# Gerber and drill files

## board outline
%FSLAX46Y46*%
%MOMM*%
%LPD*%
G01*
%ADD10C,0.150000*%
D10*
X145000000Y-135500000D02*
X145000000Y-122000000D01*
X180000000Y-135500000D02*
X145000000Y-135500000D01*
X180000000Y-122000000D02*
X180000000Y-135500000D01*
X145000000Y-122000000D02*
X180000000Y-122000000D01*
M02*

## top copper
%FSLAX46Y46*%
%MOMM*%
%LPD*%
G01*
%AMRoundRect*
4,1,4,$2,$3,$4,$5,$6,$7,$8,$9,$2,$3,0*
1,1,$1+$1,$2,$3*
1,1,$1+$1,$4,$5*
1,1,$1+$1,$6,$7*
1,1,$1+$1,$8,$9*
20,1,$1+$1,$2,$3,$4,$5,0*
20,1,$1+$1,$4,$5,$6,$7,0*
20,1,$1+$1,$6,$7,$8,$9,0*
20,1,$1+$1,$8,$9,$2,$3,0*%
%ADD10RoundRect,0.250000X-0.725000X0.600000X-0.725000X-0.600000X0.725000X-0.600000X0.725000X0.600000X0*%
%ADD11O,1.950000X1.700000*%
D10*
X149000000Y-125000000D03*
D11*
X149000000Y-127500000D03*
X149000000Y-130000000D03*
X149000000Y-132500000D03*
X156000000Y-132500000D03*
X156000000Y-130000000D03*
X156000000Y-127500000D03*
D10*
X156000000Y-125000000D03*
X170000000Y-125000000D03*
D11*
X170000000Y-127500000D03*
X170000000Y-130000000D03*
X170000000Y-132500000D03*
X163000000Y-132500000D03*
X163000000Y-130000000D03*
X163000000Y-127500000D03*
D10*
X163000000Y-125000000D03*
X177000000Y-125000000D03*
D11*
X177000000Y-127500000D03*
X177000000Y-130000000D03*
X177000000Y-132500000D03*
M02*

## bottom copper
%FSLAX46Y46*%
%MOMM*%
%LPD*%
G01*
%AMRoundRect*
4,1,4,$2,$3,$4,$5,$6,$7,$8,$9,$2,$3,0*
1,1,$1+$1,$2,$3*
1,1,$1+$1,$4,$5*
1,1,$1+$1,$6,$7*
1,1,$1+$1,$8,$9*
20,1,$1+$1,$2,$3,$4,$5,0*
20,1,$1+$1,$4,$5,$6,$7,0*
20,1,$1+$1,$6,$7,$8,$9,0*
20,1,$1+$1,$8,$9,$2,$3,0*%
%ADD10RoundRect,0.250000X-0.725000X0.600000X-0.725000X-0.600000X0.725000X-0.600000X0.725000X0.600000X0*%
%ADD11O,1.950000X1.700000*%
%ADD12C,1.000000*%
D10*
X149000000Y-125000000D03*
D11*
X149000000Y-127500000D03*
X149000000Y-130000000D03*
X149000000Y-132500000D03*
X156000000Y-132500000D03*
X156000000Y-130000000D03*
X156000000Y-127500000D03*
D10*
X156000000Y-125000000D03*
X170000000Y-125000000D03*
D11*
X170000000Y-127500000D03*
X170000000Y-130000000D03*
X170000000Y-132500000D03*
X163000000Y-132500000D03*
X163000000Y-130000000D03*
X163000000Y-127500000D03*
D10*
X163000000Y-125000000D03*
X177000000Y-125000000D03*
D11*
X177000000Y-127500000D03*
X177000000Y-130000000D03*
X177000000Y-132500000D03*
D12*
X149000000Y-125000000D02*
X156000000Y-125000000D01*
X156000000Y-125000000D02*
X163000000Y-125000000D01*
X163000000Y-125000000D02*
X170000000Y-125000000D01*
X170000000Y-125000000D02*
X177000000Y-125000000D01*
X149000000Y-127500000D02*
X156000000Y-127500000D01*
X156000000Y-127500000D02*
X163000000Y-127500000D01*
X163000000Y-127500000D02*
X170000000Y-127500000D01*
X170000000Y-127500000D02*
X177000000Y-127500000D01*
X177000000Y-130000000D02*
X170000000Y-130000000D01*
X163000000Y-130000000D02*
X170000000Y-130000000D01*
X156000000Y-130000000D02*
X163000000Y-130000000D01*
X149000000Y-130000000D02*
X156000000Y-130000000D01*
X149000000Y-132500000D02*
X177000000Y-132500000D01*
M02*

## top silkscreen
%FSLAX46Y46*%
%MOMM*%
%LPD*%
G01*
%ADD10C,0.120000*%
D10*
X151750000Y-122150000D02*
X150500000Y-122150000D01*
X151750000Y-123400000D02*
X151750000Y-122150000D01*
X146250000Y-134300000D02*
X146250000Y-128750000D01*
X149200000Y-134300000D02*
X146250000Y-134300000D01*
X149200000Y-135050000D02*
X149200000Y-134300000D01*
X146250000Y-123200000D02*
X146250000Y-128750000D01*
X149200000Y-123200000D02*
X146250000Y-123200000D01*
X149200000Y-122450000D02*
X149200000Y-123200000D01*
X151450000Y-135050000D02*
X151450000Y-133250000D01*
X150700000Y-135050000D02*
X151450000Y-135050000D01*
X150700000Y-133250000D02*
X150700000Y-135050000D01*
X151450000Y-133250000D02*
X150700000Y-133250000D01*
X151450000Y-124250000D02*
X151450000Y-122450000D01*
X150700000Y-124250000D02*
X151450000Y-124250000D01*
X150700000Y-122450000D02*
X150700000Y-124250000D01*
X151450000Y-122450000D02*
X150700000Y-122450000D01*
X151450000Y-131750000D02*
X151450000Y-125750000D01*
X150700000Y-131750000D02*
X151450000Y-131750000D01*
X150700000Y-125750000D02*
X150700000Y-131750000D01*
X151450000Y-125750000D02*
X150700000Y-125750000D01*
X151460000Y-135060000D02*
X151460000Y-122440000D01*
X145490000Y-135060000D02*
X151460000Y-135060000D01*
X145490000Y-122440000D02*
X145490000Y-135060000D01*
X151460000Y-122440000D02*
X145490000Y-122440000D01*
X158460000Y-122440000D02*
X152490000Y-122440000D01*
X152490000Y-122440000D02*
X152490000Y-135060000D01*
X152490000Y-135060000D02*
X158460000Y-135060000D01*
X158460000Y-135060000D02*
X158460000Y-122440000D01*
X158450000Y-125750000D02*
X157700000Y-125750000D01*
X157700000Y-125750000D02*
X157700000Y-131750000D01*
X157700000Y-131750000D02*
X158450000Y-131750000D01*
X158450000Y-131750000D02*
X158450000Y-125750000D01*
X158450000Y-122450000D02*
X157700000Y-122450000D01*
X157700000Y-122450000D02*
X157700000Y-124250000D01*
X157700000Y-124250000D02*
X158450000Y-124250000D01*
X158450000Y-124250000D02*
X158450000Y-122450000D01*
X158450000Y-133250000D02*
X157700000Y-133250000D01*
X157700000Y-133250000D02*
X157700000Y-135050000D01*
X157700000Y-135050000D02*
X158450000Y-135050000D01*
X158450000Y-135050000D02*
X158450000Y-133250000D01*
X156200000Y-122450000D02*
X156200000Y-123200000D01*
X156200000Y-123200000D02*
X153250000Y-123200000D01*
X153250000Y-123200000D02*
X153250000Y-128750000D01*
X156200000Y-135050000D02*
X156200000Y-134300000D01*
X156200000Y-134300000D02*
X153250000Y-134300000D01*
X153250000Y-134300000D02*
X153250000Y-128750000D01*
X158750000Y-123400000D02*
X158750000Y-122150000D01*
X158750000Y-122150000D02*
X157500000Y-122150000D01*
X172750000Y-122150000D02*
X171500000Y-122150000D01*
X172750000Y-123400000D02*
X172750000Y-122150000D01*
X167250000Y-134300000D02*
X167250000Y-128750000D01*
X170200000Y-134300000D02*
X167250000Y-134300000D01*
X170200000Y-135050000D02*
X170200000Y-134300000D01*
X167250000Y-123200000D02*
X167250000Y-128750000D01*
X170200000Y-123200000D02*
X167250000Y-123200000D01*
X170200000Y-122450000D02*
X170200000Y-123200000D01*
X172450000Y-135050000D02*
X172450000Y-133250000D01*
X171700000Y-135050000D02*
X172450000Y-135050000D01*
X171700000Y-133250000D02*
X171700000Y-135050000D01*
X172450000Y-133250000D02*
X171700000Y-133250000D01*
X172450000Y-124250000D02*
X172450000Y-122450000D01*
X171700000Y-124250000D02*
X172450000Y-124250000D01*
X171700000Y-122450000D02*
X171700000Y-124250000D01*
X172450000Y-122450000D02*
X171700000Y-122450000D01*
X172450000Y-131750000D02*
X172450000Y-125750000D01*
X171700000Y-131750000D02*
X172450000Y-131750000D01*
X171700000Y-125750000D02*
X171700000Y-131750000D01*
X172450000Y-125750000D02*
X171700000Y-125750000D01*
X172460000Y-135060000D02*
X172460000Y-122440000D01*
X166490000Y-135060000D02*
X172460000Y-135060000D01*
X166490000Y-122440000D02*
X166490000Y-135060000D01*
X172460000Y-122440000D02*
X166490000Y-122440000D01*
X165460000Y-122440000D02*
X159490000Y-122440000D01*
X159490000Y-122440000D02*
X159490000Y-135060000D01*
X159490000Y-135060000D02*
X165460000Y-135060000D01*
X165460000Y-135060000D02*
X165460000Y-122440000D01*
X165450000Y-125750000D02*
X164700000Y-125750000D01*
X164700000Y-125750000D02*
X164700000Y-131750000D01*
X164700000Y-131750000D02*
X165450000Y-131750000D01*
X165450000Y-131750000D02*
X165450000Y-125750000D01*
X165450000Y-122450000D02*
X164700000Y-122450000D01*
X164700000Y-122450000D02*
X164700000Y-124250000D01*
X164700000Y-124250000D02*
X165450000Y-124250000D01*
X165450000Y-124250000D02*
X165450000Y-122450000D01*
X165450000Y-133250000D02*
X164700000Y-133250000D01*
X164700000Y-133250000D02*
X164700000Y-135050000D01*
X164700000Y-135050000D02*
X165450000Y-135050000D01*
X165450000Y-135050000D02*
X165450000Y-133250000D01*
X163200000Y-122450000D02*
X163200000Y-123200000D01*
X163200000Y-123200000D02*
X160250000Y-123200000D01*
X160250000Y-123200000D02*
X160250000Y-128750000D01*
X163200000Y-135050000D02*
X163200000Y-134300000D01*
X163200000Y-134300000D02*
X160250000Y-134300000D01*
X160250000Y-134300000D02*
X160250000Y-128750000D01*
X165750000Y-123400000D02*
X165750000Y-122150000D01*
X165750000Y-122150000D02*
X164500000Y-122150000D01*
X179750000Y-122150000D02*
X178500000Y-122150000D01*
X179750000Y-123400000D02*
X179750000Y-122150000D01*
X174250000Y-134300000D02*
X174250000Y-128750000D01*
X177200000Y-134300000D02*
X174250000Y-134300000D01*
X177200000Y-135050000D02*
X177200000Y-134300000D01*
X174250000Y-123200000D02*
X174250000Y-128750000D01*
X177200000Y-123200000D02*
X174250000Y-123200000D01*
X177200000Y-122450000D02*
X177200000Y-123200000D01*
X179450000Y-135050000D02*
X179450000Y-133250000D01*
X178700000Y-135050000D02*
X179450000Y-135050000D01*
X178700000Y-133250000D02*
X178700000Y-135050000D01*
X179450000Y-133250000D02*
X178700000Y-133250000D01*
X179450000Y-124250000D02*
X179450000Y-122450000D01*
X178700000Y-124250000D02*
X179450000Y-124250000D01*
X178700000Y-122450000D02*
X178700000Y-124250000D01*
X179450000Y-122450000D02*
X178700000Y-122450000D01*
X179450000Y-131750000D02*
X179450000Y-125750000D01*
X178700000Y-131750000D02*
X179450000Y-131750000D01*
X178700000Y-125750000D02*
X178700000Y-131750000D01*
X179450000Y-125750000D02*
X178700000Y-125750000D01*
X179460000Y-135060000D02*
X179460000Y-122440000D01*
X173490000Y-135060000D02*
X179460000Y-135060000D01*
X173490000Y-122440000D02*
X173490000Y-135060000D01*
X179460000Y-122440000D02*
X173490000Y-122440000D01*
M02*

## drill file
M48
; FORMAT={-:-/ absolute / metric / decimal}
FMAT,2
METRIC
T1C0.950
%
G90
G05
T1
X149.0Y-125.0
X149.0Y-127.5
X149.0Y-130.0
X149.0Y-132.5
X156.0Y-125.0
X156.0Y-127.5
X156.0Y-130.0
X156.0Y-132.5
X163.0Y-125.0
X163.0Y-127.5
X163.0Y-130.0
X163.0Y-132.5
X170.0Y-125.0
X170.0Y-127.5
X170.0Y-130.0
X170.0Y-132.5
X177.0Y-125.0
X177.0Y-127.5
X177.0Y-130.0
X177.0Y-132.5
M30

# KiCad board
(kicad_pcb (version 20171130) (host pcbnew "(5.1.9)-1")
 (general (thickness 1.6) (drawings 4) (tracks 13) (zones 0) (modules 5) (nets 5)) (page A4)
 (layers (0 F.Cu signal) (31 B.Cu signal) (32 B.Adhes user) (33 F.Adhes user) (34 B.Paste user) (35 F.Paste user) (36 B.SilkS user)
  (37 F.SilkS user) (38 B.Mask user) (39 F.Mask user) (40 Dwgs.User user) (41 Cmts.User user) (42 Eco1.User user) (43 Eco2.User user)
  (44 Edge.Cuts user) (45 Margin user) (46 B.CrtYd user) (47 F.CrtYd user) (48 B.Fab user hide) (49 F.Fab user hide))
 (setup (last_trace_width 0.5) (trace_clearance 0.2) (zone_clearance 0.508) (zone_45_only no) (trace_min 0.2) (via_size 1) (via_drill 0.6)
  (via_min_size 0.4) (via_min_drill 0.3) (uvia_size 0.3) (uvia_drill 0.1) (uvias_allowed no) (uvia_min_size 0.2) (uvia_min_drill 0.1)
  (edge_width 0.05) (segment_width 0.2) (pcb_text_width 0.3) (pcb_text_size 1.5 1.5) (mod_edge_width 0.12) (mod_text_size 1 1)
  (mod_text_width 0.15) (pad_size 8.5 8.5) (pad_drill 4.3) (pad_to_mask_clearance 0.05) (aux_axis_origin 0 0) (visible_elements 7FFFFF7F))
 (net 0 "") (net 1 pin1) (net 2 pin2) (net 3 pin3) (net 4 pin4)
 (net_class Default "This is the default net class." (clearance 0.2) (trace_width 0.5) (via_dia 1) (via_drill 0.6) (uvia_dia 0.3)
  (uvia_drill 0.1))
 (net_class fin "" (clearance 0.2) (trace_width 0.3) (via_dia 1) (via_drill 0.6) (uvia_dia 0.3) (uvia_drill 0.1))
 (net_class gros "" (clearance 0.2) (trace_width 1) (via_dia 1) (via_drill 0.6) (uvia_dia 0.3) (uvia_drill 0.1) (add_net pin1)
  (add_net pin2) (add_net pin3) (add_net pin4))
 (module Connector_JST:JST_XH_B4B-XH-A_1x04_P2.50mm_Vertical (layer F.Cu) (at 149 125 270)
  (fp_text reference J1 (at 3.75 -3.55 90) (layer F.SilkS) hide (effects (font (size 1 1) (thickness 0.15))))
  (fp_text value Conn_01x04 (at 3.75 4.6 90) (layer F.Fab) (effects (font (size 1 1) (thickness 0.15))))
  (fp_line (start -2.85 -2.75) (end -2.85 -1.5) (layer F.SilkS) (width 0.12))
  (fp_line (start -1.6 -2.75) (end -2.85 -2.75) (layer F.SilkS) (width 0.12))
  (fp_line (start 9.3 2.75) (end 3.75 2.75) (layer F.SilkS) (width 0.12))
  (fp_line (start 9.3 -0.2) (end 9.3 2.75) (layer F.SilkS) (width 0.12))
  (fp_line (start 10.05 -0.2) (end 9.3 -0.2) (layer F.SilkS) (width 0.12))
  (fp_line (start -1.8 2.75) (end 3.75 2.75) (layer F.SilkS) (width 0.12))
  (fp_line (start -1.8 -0.2) (end -1.8 2.75) (layer F.SilkS) (width 0.12))
  (fp_line (start -2.55 -0.2) (end -1.8 -0.2) (layer F.SilkS) (width 0.12))
  (fp_line (start 10.05 -2.45) (end 8.25 -2.45) (layer F.SilkS) (width 0.12))
  (fp_line (start 10.05 -1.7) (end 10.05 -2.45) (layer F.SilkS) (width 0.12))
  (fp_line (start 8.25 -1.7) (end 10.05 -1.7) (layer F.SilkS) (width 0.12))
  (fp_line (start 8.25 -2.45) (end 8.25 -1.7) (layer F.SilkS) (width 0.12))
  (fp_line (start -0.75 -2.45) (end -2.55 -2.45) (layer F.SilkS) (width 0.12))
  (fp_line (start -0.75 -1.7) (end -0.75 -2.45) (layer F.SilkS) (width 0.12))
  (fp_line (start -2.55 -1.7) (end -0.75 -1.7) (layer F.SilkS) (width 0.12))
  (fp_line (start -2.55 -2.45) (end -2.55 -1.7) (layer F.SilkS) (width 0.12))
  (fp_line (start 6.75 -2.45) (end 0.75 -2.45) (layer F.SilkS) (width 0.12))
  (fp_line (start 6.75 -1.7) (end 6.75 -2.45) (layer F.SilkS) (width 0.12))
  (fp_line (start 0.75 -1.7) (end 6.75 -1.7) (layer F.SilkS) (width 0.12))
  (fp_line (start 0.75 -2.45) (end 0.75 -1.7) (layer F.SilkS) (width 0.12))
  (fp_line (start 10.06 -2.46) (end -2.56 -2.46) (layer F.SilkS) (width 0.12))
  (fp_line (start 10.06 3.51) (end 10.06 -2.46) (layer F.SilkS) (width 0.12))
  (fp_line (start -2.56 3.51) (end 10.06 3.51) (layer F.SilkS) (width 0.12))
  (fp_line (start -2.56 -2.46) (end -2.56 3.51) (layer F.SilkS) (width 0.12))
  (pad 1 thru_hole roundrect (at 0 0 270) (size 1.7 1.95) (drill 0.95) (layers *.Cu *.Mask) (roundrect_rratio 0.147059) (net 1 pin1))
  (pad 2 thru_hole oval (at 2.5 0 270) (size 1.7 1.95) (drill 0.95) (layers *.Cu *.Mask) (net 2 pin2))
  (pad 3 thru_hole oval (at 5 0 270) (size 1.7 1.95) (drill 0.95) (layers *.Cu *.Mask) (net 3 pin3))
  (pad 4 thru_hole oval (at 7.5 0 270) (size 1.7 1.95) (drill 0.95) (layers *.Cu *.Mask) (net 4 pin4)))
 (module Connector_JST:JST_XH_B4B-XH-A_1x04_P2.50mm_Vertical (layer F.Cu) (at 156 125 270)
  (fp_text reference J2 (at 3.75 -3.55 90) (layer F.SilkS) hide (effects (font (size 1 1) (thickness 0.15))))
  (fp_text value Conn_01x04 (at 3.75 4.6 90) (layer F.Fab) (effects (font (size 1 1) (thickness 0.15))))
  (fp_line (start -2.56 -2.46) (end -2.56 3.51) (layer F.SilkS) (width 0.12))
  (fp_line (start -2.56 3.51) (end 10.06 3.51) (layer F.SilkS) (width 0.12))
  (fp_line (start 10.06 3.51) (end 10.06 -2.46) (layer F.SilkS) (width 0.12))
  (fp_line (start 10.06 -2.46) (end -2.56 -2.46) (layer F.SilkS) (width 0.12))
  (fp_line (start 0.75 -2.45) (end 0.75 -1.7) (layer F.SilkS) (width 0.12))
  (fp_line (start 0.75 -1.7) (end 6.75 -1.7) (layer F.SilkS) (width 0.12))
  (fp_line (start 6.75 -1.7) (end 6.75 -2.45) (layer F.SilkS) (width 0.12))
  (fp_line (start 6.75 -2.45) (end 0.75 -2.45) (layer F.SilkS) (width 0.12))
  (fp_line (start -2.55 -2.45) (end -2.55 -1.7) (layer F.SilkS) (width 0.12))
  (fp_line (start -2.55 -1.7) (end -0.75 -1.7) (layer F.SilkS) (width 0.12))
  (fp_line (start -0.75 -1.7) (end -0.75 -2.45) (layer F.SilkS) (width 0.12))
  (fp_line (start -0.75 -2.45) (end -2.55 -2.45) (layer F.SilkS) (width 0.12))
  (fp_line (start 8.25 -2.45) (end 8.25 -1.7) (layer F.SilkS) (width 0.12))
  (fp_line (start 8.25 -1.7) (end 10.05 -1.7) (layer F.SilkS) (width 0.12))
  (fp_line (start 10.05 -1.7) (end 10.05 -2.45) (layer F.SilkS) (width 0.12))
  (fp_line (start 10.05 -2.45) (end 8.25 -2.45) (layer F.SilkS) (width 0.12))
  (fp_line (start -2.55 -0.2) (end -1.8 -0.2) (layer F.SilkS) (width 0.12))
  (fp_line (start -1.8 -0.2) (end -1.8 2.75) (layer F.SilkS) (width 0.12))
  (fp_line (start -1.8 2.75) (end 3.75 2.75) (layer F.SilkS) (width 0.12))
  (fp_line (start 10.05 -0.2) (end 9.3 -0.2) (layer F.SilkS) (width 0.12))
  (fp_line (start 9.3 -0.2) (end 9.3 2.75) (layer F.SilkS) (width 0.12))
  (fp_line (start 9.3 2.75) (end 3.75 2.75) (layer F.SilkS) (width 0.12))
  (fp_line (start -1.6 -2.75) (end -2.85 -2.75) (layer F.SilkS) (width 0.12))
  (fp_line (start -2.85 -2.75) (end -2.85 -1.5) (layer F.SilkS) (width 0.12))
  (pad 4 thru_hole oval (at 7.5 0 270) (size 1.7 1.95) (drill 0.95) (layers *.Cu *.Mask) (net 4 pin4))
  (pad 3 thru_hole oval (at 5 0 270) (size 1.7 1.95) (drill 0.95) (layers *.Cu *.Mask) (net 3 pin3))
  (pad 2 thru_hole oval (at 2.5 0 270) (size 1.7 1.95) (drill 0.95) (layers *.Cu *.Mask) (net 2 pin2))
  (pad 1 thru_hole roundrect (at 0 0 270) (size 1.7 1.95) (drill 0.95) (layers *.Cu *.Mask) (roundrect_rratio 0.147059) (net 1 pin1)))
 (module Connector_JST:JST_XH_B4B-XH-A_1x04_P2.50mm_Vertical (layer F.Cu) (at 170 125 270)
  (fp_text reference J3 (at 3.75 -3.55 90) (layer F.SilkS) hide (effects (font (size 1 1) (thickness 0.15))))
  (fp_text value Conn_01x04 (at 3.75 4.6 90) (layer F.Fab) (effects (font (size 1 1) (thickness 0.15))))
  (fp_line (start -2.85 -2.75) (end -2.85 -1.5) (layer F.SilkS) (width 0.12))
  (fp_line (start -1.6 -2.75) (end -2.85 -2.75) (layer F.SilkS) (width 0.12))
  (fp_line (start 9.3 2.75) (end 3.75 2.75) (layer F.SilkS) (width 0.12))
  (fp_line (start 9.3 -0.2) (end 9.3 2.75) (layer F.SilkS) (width 0.12))
  (fp_line (start 10.05 -0.2) (end 9.3 -0.2) (layer F.SilkS) (width 0.12))
  (fp_line (start -1.8 2.75) (end 3.75 2.75) (layer F.SilkS) (width 0.12))
  (fp_line (start -1.8 -0.2) (end -1.8 2.75) (layer F.SilkS) (width 0.12))
  (fp_line (start -2.55 -0.2) (end -1.8 -0.2) (layer F.SilkS) (width 0.12))
  (fp_line (start 10.05 -2.45) (end 8.25 -2.45) (layer F.SilkS) (width 0.12))
  (fp_line (start 10.05 -1.7) (end 10.05 -2.45) (layer F.SilkS) (width 0.12))
  (fp_line (start 8.25 -1.7) (end 10.05 -1.7) (layer F.SilkS) (width 0.12))
  (fp_line (start 8.25 -2.45) (end 8.25 -1.7) (layer F.SilkS) (width 0.12))
  (fp_line (start -0.75 -2.45) (end -2.55 -2.45) (layer F.SilkS) (width 0.12))
  (fp_line (start -0.75 -1.7) (end -0.75 -2.45) (layer F.SilkS) (width 0.12))
  (fp_line (start -2.55 -1.7) (end -0.75 -1.7) (layer F.SilkS) (width 0.12))
  (fp_line (start -2.55 -2.45) (end -2.55 -1.7) (layer F.SilkS) (width 0.12))
  (fp_line (start 6.75 -2.45) (end 0.75 -2.45) (layer F.SilkS) (width 0.12))
  (fp_line (start 6.75 -1.7) (end 6.75 -2.45) (layer F.SilkS) (width 0.12))
  (fp_line (start 0.75 -1.7) (end 6.75 -1.7) (layer F.SilkS) (width 0.12))
  (fp_line (start 0.75 -2.45) (end 0.75 -1.7) (layer F.SilkS) (width 0.12))
  (fp_line (start 10.06 -2.46) (end -2.56 -2.46) (layer F.SilkS) (width 0.12))
  (fp_line (start 10.06 3.51) (end 10.06 -2.46) (layer F.SilkS) (width 0.12))
  (fp_line (start -2.56 3.51) (end 10.06 3.51) (layer F.SilkS) (width 0.12))
  (fp_line (start -2.56 -2.46) (end -2.56 3.51) (layer F.SilkS) (width 0.12))
  (pad 1 thru_hole roundrect (at 0 0 270) (size 1.7 1.95) (drill 0.95) (layers *.Cu *.Mask) (roundrect_rratio 0.147059) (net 1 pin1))
  (pad 2 thru_hole oval (at 2.5 0 270) (size 1.7 1.95) (drill 0.95) (layers *.Cu *.Mask) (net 2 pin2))
  (pad 3 thru_hole oval (at 5 0 270) (size 1.7 1.95) (drill 0.95) (layers *.Cu *.Mask) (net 3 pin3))
  (pad 4 thru_hole oval (at 7.5 0 270) (size 1.7 1.95) (drill 0.95) (layers *.Cu *.Mask) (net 4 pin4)))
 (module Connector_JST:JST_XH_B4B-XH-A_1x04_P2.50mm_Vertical (layer F.Cu) (at 163 125 270)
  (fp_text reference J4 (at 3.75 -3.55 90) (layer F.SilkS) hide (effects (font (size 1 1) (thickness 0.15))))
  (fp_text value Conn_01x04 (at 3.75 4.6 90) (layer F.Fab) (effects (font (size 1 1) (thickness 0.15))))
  (fp_line (start -2.56 -2.46) (end -2.56 3.51) (layer F.SilkS) (width 0.12))
  (fp_line (start -2.56 3.51) (end 10.06 3.51) (layer F.SilkS) (width 0.12))
  (fp_line (start 10.06 3.51) (end 10.06 -2.46) (layer F.SilkS) (width 0.12))
  (fp_line (start 10.06 -2.46) (end -2.56 -2.46) (layer F.SilkS) (width 0.12))
  (fp_line (start 0.75 -2.45) (end 0.75 -1.7) (layer F.SilkS) (width 0.12))
  (fp_line (start 0.75 -1.7) (end 6.75 -1.7) (layer F.SilkS) (width 0.12))
  (fp_line (start 6.75 -1.7) (end 6.75 -2.45) (layer F.SilkS) (width 0.12))
  (fp_line (start 6.75 -2.45) (end 0.75 -2.45) (layer F.SilkS) (width 0.12))
  (fp_line (start -2.55 -2.45) (end -2.55 -1.7) (layer F.SilkS) (width 0.12))
  (fp_line (start -2.55 -1.7) (end -0.75 -1.7) (layer F.SilkS) (width 0.12))
  (fp_line (start -0.75 -1.7) (end -0.75 -2.45) (layer F.SilkS) (width 0.12))
  (fp_line (start -0.75 -2.45) (end -2.55 -2.45) (layer F.SilkS) (width 0.12))
  (fp_line (start 8.25 -2.45) (end 8.25 -1.7) (layer F.SilkS) (width 0.12))
  (fp_line (start 8.25 -1.7) (end 10.05 -1.7) (layer F.SilkS) (width 0.12))
  (fp_line (start 10.05 -1.7) (end 10.05 -2.45) (layer F.SilkS) (width 0.12))
  (fp_line (start 10.05 -2.45) (end 8.25 -2.45) (layer F.SilkS) (width 0.12))
  (fp_line (start -2.55 -0.2) (end -1.8 -0.2) (layer F.SilkS) (width 0.12))
  (fp_line (start -1.8 -0.2) (end -1.8 2.75) (layer F.SilkS) (width 0.12))
  (fp_line (start -1.8 2.75) (end 3.75 2.75) (layer F.SilkS) (width 0.12))
  (fp_line (start 10.05 -0.2) (end 9.3 -0.2) (layer F.SilkS) (width 0.12))
  (fp_line (start 9.3 -0.2) (end 9.3 2.75) (layer F.SilkS) (width 0.12))
  (fp_line (start 9.3 2.75) (end 3.75 2.75) (layer F.SilkS) (width 0.12))
  (fp_line (start -1.6 -2.75) (end -2.85 -2.75) (layer F.SilkS) (width 0.12))
  (fp_line (start -2.85 -2.75) (end -2.85 -1.5) (layer F.SilkS) (width 0.12))
  (pad 4 thru_hole oval (at 7.5 0 270) (size 1.7 1.95) (drill 0.95) (layers *.Cu *.Mask) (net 4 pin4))
  (pad 3 thru_hole oval (at 5 0 270) (size 1.7 1.95) (drill 0.95) (layers *.Cu *.Mask) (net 3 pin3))
  (pad 2 thru_hole oval (at 2.5 0 270) (size 1.7 1.95) (drill 0.95) (layers *.Cu *.Mask) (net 2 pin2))
  (pad 1 thru_hole roundrect (at 0 0 270) (size 1.7 1.95) (drill 0.95) (layers *.Cu *.Mask) (roundrect_rratio 0.147059) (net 1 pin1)))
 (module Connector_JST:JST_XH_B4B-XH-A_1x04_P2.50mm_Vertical (layer F.Cu) (at 177 125 270)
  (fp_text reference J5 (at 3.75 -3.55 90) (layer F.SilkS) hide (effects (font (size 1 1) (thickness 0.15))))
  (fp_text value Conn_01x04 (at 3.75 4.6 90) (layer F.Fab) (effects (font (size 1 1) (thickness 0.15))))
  (fp_line (start -2.85 -2.75) (end -2.85 -1.5) (layer F.SilkS) (width 0.12))
  (fp_line (start -1.6 -2.75) (end -2.85 -2.75) (layer F.SilkS) (width 0.12))
  (fp_line (start 9.3 2.75) (end 3.75 2.75) (layer F.SilkS) (width 0.12))
  (fp_line (start 9.3 -0.2) (end 9.3 2.75) (layer F.SilkS) (width 0.12))
  (fp_line (start 10.05 -0.2) (end 9.3 -0.2) (layer F.SilkS) (width 0.12))
  (fp_line (start -1.8 2.75) (end 3.75 2.75) (layer F.SilkS) (width 0.12))
  (fp_line (start -1.8 -0.2) (end -1.8 2.75) (layer F.SilkS) (width 0.12))
  (fp_line (start -2.55 -0.2) (end -1.8 -0.2) (layer F.SilkS) (width 0.12))
  (fp_line (start 10.05 -2.45) (end 8.25 -2.45) (layer F.SilkS) (width 0.12))
  (fp_line (start 10.05 -1.7) (end 10.05 -2.45) (layer F.SilkS) (width 0.12))
  (fp_line (start 8.25 -1.7) (end 10.05 -1.7) (layer F.SilkS) (width 0.12))
  (fp_line (start 8.25 -2.45) (end 8.25 -1.7) (layer F.SilkS) (width 0.12))
  (fp_line (start -0.75 -2.45) (end -2.55 -2.45) (layer F.SilkS) (width 0.12))
  (fp_line (start -0.75 -1.7) (end -0.75 -2.45) (layer F.SilkS) (width 0.12))
  (fp_line (start -2.55 -1.7) (end -0.75 -1.7) (layer F.SilkS) (width 0.12))
  (fp_line (start -2.55 -2.45) (end -2.55 -1.7) (layer F.SilkS) (width 0.12))
  (fp_line (start 6.75 -2.45) (end 0.75 -2.45) (layer F.SilkS) (width 0.12))
  (fp_line (start 6.75 -1.7) (end 6.75 -2.45) (layer F.SilkS) (width 0.12))
  (fp_line (start 0.75 -1.7) (end 6.75 -1.7) (layer F.SilkS) (width 0.12))
  (fp_line (start 0.75 -2.45) (end 0.75 -1.7) (layer F.SilkS) (width 0.12))
  (fp_line (start 10.06 -2.46) (end -2.56 -2.46) (layer F.SilkS) (width 0.12))
  (fp_line (start 10.06 3.51) (end 10.06 -2.46) (layer F.SilkS) (width 0.12))
  (fp_line (start -2.56 3.51) (end 10.06 3.51) (layer F.SilkS) (width 0.12))
  (fp_line (start -2.56 -2.46) (end -2.56 3.51) (layer F.SilkS) (width 0.12))
  (pad 1 thru_hole roundrect (at 0 0 270) (size 1.7 1.95) (drill 0.95) (layers *.Cu *.Mask) (roundrect_rratio 0.147059) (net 1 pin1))
  (pad 2 thru_hole oval (at 2.5 0 270) (size 1.7 1.95) (drill 0.95) (layers *.Cu *.Mask) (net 2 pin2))
  (pad 3 thru_hole oval (at 5 0 270) (size 1.7 1.95) (drill 0.95) (layers *.Cu *.Mask) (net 3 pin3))
  (pad 4 thru_hole oval (at 7.5 0 270) (size 1.7 1.95) (drill 0.95) (layers *.Cu *.Mask) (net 4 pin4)))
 (gr_line (start 145 135.5) (end 145 122) (layer Edge.Cuts) (width 0.15))
 (gr_line (start 180 135.5) (end 145 135.5) (layer Edge.Cuts) (width 0.15))
 (gr_line (start 180 122) (end 180 135.5) (layer Edge.Cuts) (width 0.15))
 (gr_line (start 145 122) (end 180 122) (layer Edge.Cuts) (width 0.15))
 (segment (start 149 125) (end 156 125) (width 1) (layer B.Cu) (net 1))
 (segment (start 156 125) (end 163 125) (width 1) (layer B.Cu) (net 1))
 (segment (start 163 125) (end 170 125) (width 1) (layer B.Cu) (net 1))
 (segment (start 170 125) (end 177 125) (width 1) (layer B.Cu) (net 1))
 (segment (start 149 127.5) (end 156 127.5) (width 1) (layer B.Cu) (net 2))
 (segment (start 156 127.5) (end 163 127.5) (width 1) (layer B.Cu) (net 2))
 (segment (start 163 127.5) (end 170 127.5) (width 1) (layer B.Cu) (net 2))
 (segment (start 170 127.5) (end 177 127.5) (width 1) (layer B.Cu) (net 2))
 (segment (start 177 130) (end 170 130) (width 1) (layer B.Cu) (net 3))
 (segment (start 163 130) (end 170 130) (width 1) (layer B.Cu) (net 3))
 (segment (start 156 130) (end 163 130) (width 1) (layer B.Cu) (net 3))
 (segment (start 149 130) (end 156 130) (width 1) (layer B.Cu) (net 3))
 (segment (start 149 132.5) (end 177 132.5) (width 1) (layer B.Cu) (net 4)))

